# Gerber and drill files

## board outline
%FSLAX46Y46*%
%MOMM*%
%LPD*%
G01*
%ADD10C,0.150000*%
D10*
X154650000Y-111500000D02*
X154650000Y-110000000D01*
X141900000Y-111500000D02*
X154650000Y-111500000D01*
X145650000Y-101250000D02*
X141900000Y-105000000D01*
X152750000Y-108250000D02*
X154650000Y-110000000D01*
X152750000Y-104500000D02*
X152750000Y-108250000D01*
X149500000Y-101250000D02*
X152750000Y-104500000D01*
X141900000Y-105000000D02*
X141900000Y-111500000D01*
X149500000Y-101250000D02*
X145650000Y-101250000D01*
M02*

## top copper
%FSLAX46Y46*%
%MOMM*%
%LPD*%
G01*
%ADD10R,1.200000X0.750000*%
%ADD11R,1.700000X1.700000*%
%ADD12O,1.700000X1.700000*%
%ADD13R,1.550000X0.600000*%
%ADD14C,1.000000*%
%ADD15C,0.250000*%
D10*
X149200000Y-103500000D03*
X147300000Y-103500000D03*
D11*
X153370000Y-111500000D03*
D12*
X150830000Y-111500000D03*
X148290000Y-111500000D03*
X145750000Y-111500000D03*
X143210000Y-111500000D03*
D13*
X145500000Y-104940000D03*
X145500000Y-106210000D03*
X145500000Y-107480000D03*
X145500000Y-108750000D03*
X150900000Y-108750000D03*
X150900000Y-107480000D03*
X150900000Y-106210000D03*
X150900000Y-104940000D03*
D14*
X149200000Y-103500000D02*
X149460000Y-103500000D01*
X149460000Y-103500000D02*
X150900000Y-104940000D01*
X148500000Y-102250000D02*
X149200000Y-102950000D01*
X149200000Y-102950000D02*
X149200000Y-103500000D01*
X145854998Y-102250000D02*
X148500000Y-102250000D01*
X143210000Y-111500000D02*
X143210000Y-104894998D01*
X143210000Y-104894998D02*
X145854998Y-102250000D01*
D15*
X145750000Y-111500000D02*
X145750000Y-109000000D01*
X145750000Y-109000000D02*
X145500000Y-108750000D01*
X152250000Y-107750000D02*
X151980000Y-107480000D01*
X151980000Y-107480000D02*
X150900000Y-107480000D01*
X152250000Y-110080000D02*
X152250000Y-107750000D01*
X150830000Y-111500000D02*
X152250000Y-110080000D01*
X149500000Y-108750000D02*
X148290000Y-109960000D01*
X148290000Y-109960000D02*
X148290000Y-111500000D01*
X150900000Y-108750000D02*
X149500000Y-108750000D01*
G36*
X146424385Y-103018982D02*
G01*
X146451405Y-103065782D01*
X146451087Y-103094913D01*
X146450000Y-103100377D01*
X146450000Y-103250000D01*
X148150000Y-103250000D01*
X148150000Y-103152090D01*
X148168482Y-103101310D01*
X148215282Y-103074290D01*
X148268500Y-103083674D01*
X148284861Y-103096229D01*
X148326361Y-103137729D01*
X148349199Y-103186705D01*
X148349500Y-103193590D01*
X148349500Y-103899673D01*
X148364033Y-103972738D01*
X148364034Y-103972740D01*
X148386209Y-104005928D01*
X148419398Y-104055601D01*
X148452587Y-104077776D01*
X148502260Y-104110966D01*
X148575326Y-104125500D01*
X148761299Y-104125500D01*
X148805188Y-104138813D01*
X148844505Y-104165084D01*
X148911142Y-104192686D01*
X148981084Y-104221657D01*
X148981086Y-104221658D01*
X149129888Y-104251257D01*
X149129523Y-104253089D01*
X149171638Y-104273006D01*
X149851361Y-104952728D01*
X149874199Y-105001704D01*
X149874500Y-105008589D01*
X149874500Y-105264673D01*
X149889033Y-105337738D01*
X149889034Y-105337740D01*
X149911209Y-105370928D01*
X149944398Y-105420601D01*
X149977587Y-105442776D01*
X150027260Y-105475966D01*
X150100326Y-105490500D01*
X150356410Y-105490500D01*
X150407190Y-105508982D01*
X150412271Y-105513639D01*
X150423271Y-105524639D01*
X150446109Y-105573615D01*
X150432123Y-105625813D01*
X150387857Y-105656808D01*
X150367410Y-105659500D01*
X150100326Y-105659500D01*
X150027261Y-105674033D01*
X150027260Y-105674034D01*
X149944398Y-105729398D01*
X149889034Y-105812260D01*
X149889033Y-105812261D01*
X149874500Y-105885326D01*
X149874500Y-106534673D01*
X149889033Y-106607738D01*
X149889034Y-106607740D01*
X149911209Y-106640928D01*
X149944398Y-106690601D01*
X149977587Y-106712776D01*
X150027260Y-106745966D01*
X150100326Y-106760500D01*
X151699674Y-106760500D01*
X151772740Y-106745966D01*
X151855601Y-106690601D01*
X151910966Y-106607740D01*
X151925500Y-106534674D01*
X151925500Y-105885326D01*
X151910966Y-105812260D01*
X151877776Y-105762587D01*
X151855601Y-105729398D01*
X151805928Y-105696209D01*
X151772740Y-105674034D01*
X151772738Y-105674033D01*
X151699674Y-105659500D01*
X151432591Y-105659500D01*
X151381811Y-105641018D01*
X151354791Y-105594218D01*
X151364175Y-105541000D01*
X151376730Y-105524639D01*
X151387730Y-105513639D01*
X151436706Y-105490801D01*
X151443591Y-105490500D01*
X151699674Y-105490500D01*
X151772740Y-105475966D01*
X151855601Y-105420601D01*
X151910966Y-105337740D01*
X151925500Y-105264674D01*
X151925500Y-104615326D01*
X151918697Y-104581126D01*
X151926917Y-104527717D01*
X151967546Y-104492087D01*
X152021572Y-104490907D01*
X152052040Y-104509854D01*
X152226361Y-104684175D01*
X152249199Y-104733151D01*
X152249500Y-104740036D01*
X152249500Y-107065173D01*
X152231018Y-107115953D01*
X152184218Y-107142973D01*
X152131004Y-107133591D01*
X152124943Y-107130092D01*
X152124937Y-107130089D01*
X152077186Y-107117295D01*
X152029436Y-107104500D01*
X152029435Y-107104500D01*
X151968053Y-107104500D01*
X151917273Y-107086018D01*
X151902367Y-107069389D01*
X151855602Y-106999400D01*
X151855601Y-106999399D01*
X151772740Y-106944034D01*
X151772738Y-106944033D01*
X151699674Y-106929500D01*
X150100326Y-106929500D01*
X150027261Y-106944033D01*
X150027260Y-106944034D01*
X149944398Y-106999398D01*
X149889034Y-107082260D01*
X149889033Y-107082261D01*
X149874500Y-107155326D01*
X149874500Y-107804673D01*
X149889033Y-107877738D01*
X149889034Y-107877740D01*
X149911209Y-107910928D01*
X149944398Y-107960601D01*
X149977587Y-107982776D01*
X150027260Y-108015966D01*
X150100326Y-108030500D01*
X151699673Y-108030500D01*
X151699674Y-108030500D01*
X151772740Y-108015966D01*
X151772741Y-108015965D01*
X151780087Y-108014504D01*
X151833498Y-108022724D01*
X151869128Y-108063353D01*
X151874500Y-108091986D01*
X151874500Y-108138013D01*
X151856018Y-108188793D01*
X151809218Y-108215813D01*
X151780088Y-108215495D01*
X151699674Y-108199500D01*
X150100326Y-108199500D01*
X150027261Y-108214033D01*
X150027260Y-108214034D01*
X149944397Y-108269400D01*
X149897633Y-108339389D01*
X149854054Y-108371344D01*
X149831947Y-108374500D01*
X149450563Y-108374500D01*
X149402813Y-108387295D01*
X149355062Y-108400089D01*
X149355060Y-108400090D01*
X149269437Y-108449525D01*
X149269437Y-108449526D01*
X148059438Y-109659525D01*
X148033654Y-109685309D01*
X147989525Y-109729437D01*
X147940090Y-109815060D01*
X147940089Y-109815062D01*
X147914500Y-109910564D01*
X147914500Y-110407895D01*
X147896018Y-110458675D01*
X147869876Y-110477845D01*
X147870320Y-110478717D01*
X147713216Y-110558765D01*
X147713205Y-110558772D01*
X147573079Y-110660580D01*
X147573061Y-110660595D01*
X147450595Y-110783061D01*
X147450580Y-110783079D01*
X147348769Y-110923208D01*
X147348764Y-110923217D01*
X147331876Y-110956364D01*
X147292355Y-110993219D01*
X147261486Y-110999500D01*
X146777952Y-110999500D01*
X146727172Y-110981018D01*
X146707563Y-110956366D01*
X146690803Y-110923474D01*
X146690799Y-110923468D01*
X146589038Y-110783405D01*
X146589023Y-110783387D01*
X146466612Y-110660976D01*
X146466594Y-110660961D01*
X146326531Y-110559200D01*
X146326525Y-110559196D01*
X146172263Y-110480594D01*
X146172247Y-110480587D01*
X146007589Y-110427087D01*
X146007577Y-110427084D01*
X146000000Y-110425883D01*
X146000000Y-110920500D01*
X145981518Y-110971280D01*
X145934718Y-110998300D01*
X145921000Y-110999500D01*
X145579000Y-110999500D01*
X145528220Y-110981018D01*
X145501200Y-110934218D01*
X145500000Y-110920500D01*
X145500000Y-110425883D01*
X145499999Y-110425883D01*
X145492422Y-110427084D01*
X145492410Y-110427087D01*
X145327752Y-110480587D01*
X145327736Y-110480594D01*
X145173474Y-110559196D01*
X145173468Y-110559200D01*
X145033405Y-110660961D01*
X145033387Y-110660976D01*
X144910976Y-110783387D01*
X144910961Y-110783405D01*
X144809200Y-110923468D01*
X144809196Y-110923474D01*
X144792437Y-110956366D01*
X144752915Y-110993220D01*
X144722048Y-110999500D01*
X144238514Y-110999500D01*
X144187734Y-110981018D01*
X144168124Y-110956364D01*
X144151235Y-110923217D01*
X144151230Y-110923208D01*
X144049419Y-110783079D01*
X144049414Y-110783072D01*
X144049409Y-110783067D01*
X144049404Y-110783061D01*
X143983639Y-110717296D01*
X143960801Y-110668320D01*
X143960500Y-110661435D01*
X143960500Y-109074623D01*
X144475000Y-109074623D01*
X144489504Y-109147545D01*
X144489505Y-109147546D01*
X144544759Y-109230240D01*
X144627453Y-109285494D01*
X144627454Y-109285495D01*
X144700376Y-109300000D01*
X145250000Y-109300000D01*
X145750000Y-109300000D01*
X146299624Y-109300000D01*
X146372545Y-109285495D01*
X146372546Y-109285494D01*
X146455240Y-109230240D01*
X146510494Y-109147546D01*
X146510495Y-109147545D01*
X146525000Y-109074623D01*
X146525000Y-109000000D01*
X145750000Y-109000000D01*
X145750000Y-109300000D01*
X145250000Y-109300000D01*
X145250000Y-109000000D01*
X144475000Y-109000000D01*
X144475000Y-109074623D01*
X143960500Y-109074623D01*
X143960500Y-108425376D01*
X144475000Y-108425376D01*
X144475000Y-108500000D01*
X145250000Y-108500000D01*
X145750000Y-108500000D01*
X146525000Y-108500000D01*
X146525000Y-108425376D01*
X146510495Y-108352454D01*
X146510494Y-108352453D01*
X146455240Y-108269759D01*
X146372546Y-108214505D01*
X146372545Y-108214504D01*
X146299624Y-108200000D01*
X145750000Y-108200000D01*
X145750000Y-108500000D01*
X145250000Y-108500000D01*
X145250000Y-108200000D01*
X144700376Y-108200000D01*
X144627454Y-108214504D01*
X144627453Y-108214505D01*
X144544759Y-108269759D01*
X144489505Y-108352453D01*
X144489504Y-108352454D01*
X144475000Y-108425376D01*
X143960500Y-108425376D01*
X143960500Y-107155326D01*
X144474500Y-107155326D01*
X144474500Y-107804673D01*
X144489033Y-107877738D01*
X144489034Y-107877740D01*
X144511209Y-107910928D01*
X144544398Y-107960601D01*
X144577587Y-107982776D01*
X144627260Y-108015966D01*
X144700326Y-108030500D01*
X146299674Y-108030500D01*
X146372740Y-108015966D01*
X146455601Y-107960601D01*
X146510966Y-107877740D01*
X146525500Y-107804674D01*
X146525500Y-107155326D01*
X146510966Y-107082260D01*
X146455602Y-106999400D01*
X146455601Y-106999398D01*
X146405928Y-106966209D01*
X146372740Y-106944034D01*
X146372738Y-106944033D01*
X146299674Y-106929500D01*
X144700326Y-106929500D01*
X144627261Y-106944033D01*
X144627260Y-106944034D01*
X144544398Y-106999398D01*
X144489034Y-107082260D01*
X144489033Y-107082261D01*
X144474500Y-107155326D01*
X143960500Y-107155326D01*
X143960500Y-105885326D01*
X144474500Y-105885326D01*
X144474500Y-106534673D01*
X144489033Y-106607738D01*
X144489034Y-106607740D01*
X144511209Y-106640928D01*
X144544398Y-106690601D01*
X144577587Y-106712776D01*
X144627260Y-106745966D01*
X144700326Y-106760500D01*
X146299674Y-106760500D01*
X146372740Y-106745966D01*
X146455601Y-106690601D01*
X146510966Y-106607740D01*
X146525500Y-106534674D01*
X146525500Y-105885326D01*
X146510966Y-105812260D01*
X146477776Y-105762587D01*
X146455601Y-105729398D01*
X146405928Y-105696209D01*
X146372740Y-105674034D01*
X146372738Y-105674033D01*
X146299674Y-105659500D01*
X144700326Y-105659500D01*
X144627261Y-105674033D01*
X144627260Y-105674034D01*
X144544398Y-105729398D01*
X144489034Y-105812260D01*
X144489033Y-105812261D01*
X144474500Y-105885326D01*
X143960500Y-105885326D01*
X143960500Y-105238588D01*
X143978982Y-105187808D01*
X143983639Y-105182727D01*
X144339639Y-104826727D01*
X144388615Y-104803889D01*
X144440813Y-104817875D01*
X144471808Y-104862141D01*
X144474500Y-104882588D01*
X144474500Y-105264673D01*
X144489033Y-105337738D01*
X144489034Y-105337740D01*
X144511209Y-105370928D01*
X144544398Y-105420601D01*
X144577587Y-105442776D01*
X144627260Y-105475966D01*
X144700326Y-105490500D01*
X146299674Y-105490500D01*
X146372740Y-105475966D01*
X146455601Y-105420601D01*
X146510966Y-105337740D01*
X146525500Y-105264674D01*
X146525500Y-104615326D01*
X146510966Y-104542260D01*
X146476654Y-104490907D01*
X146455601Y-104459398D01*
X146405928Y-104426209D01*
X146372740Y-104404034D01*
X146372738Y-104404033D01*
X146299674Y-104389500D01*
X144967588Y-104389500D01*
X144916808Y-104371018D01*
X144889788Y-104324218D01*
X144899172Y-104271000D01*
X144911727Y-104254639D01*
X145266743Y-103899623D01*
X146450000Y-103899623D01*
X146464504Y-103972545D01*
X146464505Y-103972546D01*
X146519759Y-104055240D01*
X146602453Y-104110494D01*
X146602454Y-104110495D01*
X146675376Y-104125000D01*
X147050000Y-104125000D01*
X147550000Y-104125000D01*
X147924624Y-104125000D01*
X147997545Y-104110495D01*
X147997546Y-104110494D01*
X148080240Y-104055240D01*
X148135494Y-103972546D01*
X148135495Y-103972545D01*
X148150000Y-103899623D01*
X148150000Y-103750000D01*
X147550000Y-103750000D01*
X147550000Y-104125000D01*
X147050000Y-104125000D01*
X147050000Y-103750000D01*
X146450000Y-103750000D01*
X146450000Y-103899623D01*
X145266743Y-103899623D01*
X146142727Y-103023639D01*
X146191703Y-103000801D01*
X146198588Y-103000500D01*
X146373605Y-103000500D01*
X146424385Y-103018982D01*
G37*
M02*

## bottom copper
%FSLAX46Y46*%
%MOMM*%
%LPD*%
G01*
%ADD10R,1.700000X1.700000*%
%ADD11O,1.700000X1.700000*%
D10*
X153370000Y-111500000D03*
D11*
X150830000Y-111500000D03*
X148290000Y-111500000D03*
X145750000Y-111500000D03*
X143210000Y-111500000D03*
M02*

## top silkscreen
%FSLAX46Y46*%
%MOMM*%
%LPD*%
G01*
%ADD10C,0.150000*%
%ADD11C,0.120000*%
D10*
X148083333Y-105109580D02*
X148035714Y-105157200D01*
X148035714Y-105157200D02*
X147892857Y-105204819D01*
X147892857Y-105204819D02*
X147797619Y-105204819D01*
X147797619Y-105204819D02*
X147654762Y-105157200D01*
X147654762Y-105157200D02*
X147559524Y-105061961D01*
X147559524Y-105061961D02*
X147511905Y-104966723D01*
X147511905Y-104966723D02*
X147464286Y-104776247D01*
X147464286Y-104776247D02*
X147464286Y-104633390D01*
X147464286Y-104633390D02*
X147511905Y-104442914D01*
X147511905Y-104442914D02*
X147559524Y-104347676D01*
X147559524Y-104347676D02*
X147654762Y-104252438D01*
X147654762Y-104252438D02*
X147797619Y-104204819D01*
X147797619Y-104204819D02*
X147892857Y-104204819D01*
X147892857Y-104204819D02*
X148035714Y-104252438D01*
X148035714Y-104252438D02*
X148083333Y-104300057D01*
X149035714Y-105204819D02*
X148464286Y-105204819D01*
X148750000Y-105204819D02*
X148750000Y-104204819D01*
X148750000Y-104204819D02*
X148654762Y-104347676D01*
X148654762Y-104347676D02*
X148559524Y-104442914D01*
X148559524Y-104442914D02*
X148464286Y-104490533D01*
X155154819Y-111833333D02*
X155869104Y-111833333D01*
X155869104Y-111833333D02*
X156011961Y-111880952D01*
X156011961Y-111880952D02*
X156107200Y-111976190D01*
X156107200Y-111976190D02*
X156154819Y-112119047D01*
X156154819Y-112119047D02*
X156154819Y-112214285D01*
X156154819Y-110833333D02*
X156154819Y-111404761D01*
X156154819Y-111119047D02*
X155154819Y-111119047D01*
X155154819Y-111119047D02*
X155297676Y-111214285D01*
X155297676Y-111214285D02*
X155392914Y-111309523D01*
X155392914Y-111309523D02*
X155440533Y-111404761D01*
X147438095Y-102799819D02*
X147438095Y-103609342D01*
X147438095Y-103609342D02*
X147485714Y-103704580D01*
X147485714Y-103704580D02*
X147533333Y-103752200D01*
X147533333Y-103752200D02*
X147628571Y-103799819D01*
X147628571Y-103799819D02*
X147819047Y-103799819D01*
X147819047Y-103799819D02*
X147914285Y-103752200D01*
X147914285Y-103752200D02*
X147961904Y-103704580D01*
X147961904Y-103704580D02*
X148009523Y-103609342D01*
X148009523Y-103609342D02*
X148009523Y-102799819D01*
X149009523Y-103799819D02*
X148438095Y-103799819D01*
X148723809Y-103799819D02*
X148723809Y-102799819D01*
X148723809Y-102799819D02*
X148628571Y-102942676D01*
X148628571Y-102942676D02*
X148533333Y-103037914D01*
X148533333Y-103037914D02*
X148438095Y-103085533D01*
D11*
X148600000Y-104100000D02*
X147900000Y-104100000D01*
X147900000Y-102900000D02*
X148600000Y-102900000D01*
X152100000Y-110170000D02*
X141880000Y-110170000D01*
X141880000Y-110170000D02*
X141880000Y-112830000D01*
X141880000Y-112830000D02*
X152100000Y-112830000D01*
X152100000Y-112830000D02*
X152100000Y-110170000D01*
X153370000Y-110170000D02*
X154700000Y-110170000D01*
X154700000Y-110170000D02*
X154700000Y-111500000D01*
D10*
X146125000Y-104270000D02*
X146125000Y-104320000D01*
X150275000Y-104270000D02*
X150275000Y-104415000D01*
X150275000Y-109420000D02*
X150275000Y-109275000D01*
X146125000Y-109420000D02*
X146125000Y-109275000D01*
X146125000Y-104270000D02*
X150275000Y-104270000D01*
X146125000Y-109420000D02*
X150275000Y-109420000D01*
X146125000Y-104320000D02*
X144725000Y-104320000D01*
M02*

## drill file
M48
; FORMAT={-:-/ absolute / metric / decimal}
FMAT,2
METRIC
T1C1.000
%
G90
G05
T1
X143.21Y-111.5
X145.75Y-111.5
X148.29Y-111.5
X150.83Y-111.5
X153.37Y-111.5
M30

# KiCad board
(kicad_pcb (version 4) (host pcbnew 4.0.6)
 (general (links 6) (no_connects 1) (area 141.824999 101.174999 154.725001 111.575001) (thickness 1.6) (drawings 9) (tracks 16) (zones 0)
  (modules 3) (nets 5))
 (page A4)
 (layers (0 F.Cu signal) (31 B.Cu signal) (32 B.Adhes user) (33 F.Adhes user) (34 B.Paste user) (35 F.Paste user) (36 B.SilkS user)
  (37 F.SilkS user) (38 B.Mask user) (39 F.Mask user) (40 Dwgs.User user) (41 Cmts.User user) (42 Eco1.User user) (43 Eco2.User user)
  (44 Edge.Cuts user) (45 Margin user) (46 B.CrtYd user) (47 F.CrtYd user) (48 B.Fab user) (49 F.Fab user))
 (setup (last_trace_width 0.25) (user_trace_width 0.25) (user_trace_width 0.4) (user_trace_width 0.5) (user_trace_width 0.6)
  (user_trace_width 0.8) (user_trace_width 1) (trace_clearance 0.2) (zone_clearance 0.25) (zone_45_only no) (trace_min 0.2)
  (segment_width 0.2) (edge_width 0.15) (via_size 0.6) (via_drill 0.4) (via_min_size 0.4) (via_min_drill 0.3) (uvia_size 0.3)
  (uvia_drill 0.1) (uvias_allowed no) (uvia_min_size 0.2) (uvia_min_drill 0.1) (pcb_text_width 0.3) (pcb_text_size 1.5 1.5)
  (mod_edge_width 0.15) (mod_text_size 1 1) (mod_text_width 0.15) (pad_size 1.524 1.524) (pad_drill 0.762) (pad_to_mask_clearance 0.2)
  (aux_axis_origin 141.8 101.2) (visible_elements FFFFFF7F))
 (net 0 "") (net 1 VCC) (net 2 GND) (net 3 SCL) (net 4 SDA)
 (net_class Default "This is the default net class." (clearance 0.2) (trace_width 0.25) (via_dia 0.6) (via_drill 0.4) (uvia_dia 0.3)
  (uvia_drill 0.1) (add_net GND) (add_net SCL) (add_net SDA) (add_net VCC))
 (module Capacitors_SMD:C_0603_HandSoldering (layer F.Cu) (at 148.25 103.5 180)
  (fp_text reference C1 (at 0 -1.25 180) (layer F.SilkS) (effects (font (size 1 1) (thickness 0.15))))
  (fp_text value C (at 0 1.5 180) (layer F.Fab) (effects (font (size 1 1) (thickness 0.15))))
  (fp_line (start -0.35 -0.6) (end 0.35 -0.6) (layer F.SilkS) (width 0.12))
  (fp_line (start 0.35 0.6) (end -0.35 0.6) (layer F.SilkS) (width 0.12))
  (pad 1 smd rect (at -0.95 0 180) (size 1.2 0.75) (layers F.Cu F.Paste F.Mask) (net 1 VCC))
  (pad 2 smd rect (at 0.95 0 180) (size 1.2 0.75) (layers F.Cu F.Paste F.Mask) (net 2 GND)))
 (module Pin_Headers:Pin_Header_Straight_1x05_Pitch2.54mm (layer F.Cu) (at 153.37 111.5 270)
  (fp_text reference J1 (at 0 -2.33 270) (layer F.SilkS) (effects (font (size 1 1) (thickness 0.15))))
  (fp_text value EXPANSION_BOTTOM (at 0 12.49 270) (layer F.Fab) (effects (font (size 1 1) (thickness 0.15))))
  (fp_line (start -1.33 1.27) (end -1.33 11.49) (layer F.SilkS) (width 0.12))
  (fp_line (start -1.33 11.49) (end 1.33 11.49) (layer F.SilkS) (width 0.12))
  (fp_line (start 1.33 11.49) (end 1.33 1.27) (layer F.SilkS) (width 0.12))
  (fp_line (start 1.33 1.27) (end -1.33 1.27) (layer F.SilkS) (width 0.12))
  (fp_line (start -1.33 0) (end -1.33 -1.33) (layer F.SilkS) (width 0.12))
  (fp_line (start -1.33 -1.33) (end 0 -1.33) (layer F.SilkS) (width 0.12))
  (pad 1 thru_hole rect (at 0 0 270) (size 1.7 1.7) (drill 1) (layers *.Cu *.Mask))
  (pad 2 thru_hole oval (at 0 2.54 270) (size 1.7 1.7) (drill 1) (layers *.Cu *.Mask) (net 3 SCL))
  (pad 3 thru_hole oval (at 0 5.08 270) (size 1.7 1.7) (drill 1) (layers *.Cu *.Mask) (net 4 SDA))
  (pad 4 thru_hole oval (at 0 7.62 270) (size 1.7 1.7) (drill 1) (layers *.Cu *.Mask) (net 2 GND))
  (pad 5 thru_hole oval (at 0 10.16 270) (size 1.7 1.7) (drill 1) (layers *.Cu *.Mask) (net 1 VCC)))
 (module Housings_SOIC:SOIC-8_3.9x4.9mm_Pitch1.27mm (layer F.Cu) (at 148.2 106.845)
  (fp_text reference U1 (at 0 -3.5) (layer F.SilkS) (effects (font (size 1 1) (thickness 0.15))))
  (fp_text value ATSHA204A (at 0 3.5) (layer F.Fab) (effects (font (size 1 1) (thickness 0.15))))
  (fp_line (start -2.075 -2.575) (end -2.075 -2.525) (layer F.SilkS) (width 0.15))
  (fp_line (start 2.075 -2.575) (end 2.075 -2.43) (layer F.SilkS) (width 0.15))
  (fp_line (start 2.075 2.575) (end 2.075 2.43) (layer F.SilkS) (width 0.15))
  (fp_line (start -2.075 2.575) (end -2.075 2.43) (layer F.SilkS) (width 0.15))
  (fp_line (start -2.075 -2.575) (end 2.075 -2.575) (layer F.SilkS) (width 0.15))
  (fp_line (start -2.075 2.575) (end 2.075 2.575) (layer F.SilkS) (width 0.15))
  (fp_line (start -2.075 -2.525) (end -3.475 -2.525) (layer F.SilkS) (width 0.15))
  (pad 1 smd rect (at -2.7 -1.905) (size 1.55 0.6) (layers F.Cu F.Paste F.Mask))
  (pad 2 smd rect (at -2.7 -0.635) (size 1.55 0.6) (layers F.Cu F.Paste F.Mask))
  (pad 3 smd rect (at -2.7 0.635) (size 1.55 0.6) (layers F.Cu F.Paste F.Mask))
  (pad 4 smd rect (at -2.7 1.905) (size 1.55 0.6) (layers F.Cu F.Paste F.Mask) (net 2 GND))
  (pad 5 smd rect (at 2.7 1.905) (size 1.55 0.6) (layers F.Cu F.Paste F.Mask) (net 4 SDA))
  (pad 6 smd rect (at 2.7 0.635) (size 1.55 0.6) (layers F.Cu F.Paste F.Mask) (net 3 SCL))
  (pad 7 smd rect (at 2.7 -0.635) (size 1.55 0.6) (layers F.Cu F.Paste F.Mask))
  (pad 8 smd rect (at 2.7 -1.905) (size 1.55 0.6) (layers F.Cu F.Paste F.Mask) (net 1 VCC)))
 (gr_line (start 154.65 111.5) (end 154.65 110) (layer Edge.Cuts) (width 0.15))
 (gr_line (start 141.9 111.5) (end 154.65 111.5) (layer Edge.Cuts) (width 0.15))
 (gr_line (start 145.65 101.25) (end 141.9 105) (layer Edge.Cuts) (width 0.15))
 (gr_line (start 152.75 108.25) (end 154.65 110) (layer Edge.Cuts) (width 0.15))
 (gr_line (start 152.75 104.5) (end 152.75 108.25) (layer Edge.Cuts) (width 0.15))
 (gr_line (start 149.5 101.25) (end 152.75 104.5) (layer Edge.Cuts) (width 0.15))
 (gr_line (start 141.9 105) (end 141.9 111.5) (layer Edge.Cuts) (width 0.15))
 (gr_line (start 149.5 101.25) (end 145.65 101.25) (layer Edge.Cuts) (width 0.15))
 (segment (start 149.2 103.5) (end 149.46 103.5) (width 1) (layer F.Cu) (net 1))
 (segment (start 149.46 103.5) (end 150.9 104.94) (width 1) (layer F.Cu) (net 1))
 (segment (start 148.5 102.25) (end 149.2 102.95) (width 1) (layer F.Cu) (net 1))
 (segment (start 149.2 102.95) (end 149.2 103.5) (width 1) (layer F.Cu) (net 1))
 (segment (start 145.854998 102.25) (end 148.5 102.25) (width 1) (layer F.Cu) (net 1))
 (segment (start 143.21 111.5) (end 143.21 104.894998) (width 1) (layer F.Cu) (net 1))
 (segment (start 143.21 104.894998) (end 145.854998 102.25) (width 1) (layer F.Cu) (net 1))
 (segment (start 145.75 111.5) (end 145.75 109) (width 0.25) (layer F.Cu) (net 2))
 (segment (start 145.75 109) (end 145.5 108.75) (width 0.25) (layer F.Cu) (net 2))
 (segment (start 152.25 107.75) (end 151.98 107.48) (width 0.25) (layer F.Cu) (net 3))
 (segment (start 151.98 107.48) (end 150.9 107.48) (width 0.25) (layer F.Cu) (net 3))
 (segment (start 152.25 110.08) (end 152.25 107.75) (width 0.25) (layer F.Cu) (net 3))
 (segment (start 150.83 111.5) (end 152.25 110.08) (width 0.25) (layer F.Cu) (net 3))
 (segment (start 149.5 108.75) (end 148.29 109.96) (width 0.25) (layer F.Cu) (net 4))
 (segment (start 148.29 109.96) (end 148.29 111.5) (width 0.25) (layer F.Cu) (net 4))
 (segment (start 150.9 108.75) (end 149.5 108.75) (width 0.25) (layer F.Cu) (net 4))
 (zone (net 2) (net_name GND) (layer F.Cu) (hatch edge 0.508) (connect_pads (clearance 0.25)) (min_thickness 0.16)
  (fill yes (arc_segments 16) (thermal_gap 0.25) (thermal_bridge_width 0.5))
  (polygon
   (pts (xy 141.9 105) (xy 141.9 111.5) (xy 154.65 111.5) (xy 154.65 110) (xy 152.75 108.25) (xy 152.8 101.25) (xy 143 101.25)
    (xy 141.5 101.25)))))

